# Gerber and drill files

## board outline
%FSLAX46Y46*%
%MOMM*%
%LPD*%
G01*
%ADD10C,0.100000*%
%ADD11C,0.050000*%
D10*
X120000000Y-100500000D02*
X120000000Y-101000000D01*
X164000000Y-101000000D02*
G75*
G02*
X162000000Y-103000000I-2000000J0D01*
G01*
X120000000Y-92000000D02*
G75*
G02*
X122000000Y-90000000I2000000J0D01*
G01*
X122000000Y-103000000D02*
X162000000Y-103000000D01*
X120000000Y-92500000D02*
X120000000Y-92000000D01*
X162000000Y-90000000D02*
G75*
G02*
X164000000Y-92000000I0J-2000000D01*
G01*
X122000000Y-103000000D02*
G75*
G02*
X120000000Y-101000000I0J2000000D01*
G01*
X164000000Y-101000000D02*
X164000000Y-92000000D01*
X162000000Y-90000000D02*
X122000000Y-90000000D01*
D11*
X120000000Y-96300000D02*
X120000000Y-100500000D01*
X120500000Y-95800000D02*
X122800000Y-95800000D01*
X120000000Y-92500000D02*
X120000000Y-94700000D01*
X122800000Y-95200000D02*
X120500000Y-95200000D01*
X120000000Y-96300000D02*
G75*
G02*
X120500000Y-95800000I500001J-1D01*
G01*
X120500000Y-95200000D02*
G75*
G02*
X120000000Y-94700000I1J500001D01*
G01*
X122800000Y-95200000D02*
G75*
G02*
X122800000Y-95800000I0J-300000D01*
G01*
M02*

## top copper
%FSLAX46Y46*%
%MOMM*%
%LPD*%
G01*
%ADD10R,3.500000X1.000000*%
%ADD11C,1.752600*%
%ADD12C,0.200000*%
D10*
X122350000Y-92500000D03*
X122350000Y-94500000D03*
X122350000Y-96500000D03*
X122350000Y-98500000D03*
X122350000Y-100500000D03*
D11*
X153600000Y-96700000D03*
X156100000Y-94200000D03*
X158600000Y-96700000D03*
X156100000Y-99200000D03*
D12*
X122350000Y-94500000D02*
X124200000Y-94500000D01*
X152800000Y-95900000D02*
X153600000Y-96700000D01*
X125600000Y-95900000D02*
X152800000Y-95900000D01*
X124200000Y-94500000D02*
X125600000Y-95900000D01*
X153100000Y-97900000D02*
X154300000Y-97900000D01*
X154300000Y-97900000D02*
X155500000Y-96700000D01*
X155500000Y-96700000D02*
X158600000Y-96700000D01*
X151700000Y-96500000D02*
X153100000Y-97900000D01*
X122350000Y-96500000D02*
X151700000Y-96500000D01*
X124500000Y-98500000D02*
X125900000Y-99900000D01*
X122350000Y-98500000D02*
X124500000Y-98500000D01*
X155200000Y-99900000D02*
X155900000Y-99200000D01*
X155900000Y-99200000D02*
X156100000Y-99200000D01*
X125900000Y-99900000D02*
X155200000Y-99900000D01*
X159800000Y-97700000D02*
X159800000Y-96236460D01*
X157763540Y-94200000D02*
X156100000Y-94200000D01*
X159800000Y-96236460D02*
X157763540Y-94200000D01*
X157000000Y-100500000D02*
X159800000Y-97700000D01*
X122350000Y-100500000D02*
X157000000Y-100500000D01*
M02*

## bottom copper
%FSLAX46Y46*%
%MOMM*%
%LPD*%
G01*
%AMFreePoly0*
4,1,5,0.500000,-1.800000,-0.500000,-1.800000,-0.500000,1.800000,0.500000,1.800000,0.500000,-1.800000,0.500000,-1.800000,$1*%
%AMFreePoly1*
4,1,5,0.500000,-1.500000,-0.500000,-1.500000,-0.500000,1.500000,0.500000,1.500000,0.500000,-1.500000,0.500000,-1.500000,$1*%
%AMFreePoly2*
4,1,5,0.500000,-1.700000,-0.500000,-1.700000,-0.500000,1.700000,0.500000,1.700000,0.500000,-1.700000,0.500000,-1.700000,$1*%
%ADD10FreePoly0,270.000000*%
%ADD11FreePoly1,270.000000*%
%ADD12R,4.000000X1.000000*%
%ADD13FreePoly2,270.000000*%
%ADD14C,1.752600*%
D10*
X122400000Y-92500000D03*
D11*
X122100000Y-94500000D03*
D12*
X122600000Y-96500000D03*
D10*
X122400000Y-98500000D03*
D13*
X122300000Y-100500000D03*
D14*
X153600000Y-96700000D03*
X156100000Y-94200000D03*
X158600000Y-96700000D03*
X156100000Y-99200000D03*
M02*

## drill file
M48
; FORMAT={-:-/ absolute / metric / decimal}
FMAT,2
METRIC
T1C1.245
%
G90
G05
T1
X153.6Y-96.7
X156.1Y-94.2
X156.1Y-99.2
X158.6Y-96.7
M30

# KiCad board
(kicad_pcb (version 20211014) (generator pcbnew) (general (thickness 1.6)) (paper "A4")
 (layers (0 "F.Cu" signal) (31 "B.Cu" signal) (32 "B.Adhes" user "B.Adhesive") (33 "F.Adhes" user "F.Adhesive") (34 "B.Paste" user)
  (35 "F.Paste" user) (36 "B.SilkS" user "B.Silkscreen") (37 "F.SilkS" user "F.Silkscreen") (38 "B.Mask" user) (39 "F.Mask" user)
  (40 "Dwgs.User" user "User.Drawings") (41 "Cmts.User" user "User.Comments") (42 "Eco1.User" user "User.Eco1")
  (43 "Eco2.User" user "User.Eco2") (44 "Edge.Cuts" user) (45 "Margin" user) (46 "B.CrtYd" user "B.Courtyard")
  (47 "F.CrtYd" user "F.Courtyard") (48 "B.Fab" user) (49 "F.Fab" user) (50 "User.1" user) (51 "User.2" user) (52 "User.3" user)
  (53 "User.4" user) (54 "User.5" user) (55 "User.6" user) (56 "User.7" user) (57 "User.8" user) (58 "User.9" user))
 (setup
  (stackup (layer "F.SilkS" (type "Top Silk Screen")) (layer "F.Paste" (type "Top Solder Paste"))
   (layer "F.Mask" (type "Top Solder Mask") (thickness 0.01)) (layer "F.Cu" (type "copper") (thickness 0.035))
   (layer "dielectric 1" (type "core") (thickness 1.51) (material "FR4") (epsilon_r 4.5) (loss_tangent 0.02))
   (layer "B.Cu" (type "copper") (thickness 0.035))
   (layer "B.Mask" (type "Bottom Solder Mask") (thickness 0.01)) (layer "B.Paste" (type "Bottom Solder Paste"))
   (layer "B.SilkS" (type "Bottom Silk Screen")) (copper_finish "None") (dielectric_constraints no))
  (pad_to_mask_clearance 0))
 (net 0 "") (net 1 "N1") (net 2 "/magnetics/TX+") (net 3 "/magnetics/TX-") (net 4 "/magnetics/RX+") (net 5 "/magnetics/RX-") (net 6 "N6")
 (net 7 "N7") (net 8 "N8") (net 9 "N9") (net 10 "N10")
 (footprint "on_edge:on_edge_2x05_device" (layer "F.Cu") (at 120 96.5 -90)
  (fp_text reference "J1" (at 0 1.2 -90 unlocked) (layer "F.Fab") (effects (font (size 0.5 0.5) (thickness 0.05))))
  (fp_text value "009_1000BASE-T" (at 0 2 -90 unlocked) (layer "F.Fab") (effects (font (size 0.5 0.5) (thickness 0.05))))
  (fp_line (start -0.2 0) (end 4 0) (layer "Edge.Cuts") (width 0.05))
  (fp_line (start -0.7 -0.5) (end -0.7 -2.8) (layer "Edge.Cuts") (width 0.05))
  (fp_line (start -4 0) (end -1.8 0) (layer "Edge.Cuts") (width 0.05))
  (fp_line (start -1.3 -2.8) (end -1.3 -0.5) (layer "Edge.Cuts") (width 0.05))
  (fp_arc (start -0.2 0) (mid -0.553553 -0.146447) (end -0.7 -0.5) (layer "Edge.Cuts") (width 0.05))
  (fp_arc (start -1.3 -0.5) (mid -1.446447 -0.146447) (end -1.8 0) (layer "Edge.Cuts") (width 0.05))
  (fp_arc (start -1.3 -2.8) (mid -1 -3.1) (end -0.7 -2.8) (layer "Edge.Cuts") (width 0.05))
  (pad "1" smd rect (at -4 -2.35 90) (size 1 3.5) (layers "F.Cu" "F.Mask") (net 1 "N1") (zone_connect 0))
  (pad "2" smd rect (at -2 -2.35 270) (size 1 3.5) (layers "F.Cu" "F.Mask") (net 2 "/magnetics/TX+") (zone_connect 0))
  (pad "3" smd rect (at 0 -2.35 270) (size 1 3.5) (layers "F.Cu" "F.Mask") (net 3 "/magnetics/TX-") (zone_connect 0))
  (pad "4" smd rect (at 2 -2.35 90) (size 1 3.5) (layers "F.Cu" "F.Mask") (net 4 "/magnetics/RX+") (zone_connect 0))
  (pad "5" smd rect (at 4 -2.35 90) (size 1 3.5) (layers "F.Cu" "F.Mask") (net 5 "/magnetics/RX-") (zone_connect 0))
  (pad "6" smd custom (at -4 -2.4 270) (size 1 3.6) (layers "B.Cu" "B.Mask") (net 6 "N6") (zone_connect 0)
   (options (clearance outline) (anchor rect)) (primitives))
  (pad "7" smd custom (at -2 -2.1 270) (size 1 3) (layers "B.Cu" "B.Mask") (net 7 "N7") (zone_connect 0)
   (options (clearance outline) (anchor rect)) (primitives))
  (pad "8" smd rect (at 0 -2.6 270) (size 1 4) (layers "B.Cu" "B.Mask") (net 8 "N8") (zone_connect 0))
  (pad "9" smd custom (at 2 -2.4 270) (size 1 3.6) (layers "B.Cu" "B.Mask") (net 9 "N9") (zone_connect 0)
   (options (clearance outline) (anchor rect)) (primitives))
  (pad "10" smd custom (at 4 -2.3 270) (size 1 3.4) (layers "B.Cu" "B.Mask") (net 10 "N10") (zone_connect 0)
   (options (clearance outline) (anchor rect)) (primitives)))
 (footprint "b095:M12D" (layer "F.Cu") (at 156.1 96.7)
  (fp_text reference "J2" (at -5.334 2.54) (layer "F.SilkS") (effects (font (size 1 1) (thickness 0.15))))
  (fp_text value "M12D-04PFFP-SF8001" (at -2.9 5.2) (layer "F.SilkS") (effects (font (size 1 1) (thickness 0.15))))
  (pad "1" thru_hole circle (at -2.5 0) (size 1.7526 1.7526) (drill 1.2446) (layers *.Cu *.Mask) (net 2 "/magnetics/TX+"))
  (pad "2" thru_hole circle (at 0 -2.5) (size 1.7526 1.7526) (drill 1.2446) (layers *.Cu *.Mask) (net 5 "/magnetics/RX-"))
  (pad "3" thru_hole circle (at 2.5 0 90) (size 1.7526 1.7526) (drill 1.2446) (layers *.Cu *.Mask) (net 3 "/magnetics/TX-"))
  (pad "4" thru_hole circle (at 0 2.5 90) (size 1.7526 1.7526) (drill 1.2446) (layers *.Cu *.Mask) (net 4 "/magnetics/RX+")))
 (gr_line (start 120 100.5) (end 120 101) (layer "Edge.Cuts") (width 0.1))
 (gr_arc (start 164 101) (mid 163.414214 102.414214) (end 162 103) (layer "Edge.Cuts") (width 0.1))
 (gr_arc (start 120 92) (mid 120.585786 90.585786) (end 122 90) (layer "Edge.Cuts") (width 0.1))
 (gr_line (start 122 103) (end 162 103) (layer "Edge.Cuts") (width 0.1))
 (gr_line (start 120 92.5) (end 120 92) (layer "Edge.Cuts") (width 0.1))
 (gr_arc (start 162 90) (mid 163.414214 90.585786) (end 164 92) (layer "Edge.Cuts") (width 0.1))
 (gr_arc (start 122 103) (mid 120.585786 102.414214) (end 120 101) (layer "Edge.Cuts") (width 0.1))
 (gr_line (start 164 101) (end 164 92) (layer "Edge.Cuts") (width 0.1))
 (gr_line (start 162 90) (end 122 90) (layer "Edge.Cuts") (width 0.1))
 (segment (start 122.35 94.5) (end 124.2 94.5) (width 0.2) (layer "F.Cu") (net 2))
 (segment (start 152.8 95.9) (end 153.6 96.7) (width 0.2) (layer "F.Cu") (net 2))
 (segment (start 125.6 95.9) (end 152.8 95.9) (width 0.2) (layer "F.Cu") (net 2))
 (segment (start 124.2 94.5) (end 125.6 95.9) (width 0.2) (layer "F.Cu") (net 2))
 (segment (start 153.1 97.9) (end 154.3 97.9) (width 0.2) (layer "F.Cu") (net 3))
 (segment (start 154.3 97.9) (end 155.5 96.7) (width 0.2) (layer "F.Cu") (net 3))
 (segment (start 155.5 96.7) (end 158.6 96.7) (width 0.2) (layer "F.Cu") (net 3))
 (segment (start 151.7 96.5) (end 153.1 97.9) (width 0.2) (layer "F.Cu") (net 3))
 (segment (start 122.35 96.5) (end 151.7 96.5) (width 0.2) (layer "F.Cu") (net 3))
 (segment (start 124.5 98.5) (end 125.9 99.9) (width 0.2) (layer "F.Cu") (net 4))
 (segment (start 122.35 98.5) (end 124.5 98.5) (width 0.2) (layer "F.Cu") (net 4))
 (segment (start 155.2 99.9) (end 155.9 99.2) (width 0.2) (layer "F.Cu") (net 4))
 (segment (start 155.9 99.2) (end 156.1 99.2) (width 0.2) (layer "F.Cu") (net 4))
 (segment (start 125.9 99.9) (end 155.2 99.9) (width 0.2) (layer "F.Cu") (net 4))
 (segment (start 159.8 97.7) (end 159.8 96.23646) (width 0.2) (layer "F.Cu") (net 5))
 (segment (start 157.76354 94.2) (end 156.1 94.2) (width 0.2) (layer "F.Cu") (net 5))
 (segment (start 159.8 96.23646) (end 157.76354 94.2) (width 0.2) (layer "F.Cu") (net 5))
 (segment (start 157 100.5) (end 159.8 97.7) (width 0.2) (layer "F.Cu") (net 5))
 (segment (start 122.35 100.5) (end 157 100.5) (width 0.2) (layer "F.Cu") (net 5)))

